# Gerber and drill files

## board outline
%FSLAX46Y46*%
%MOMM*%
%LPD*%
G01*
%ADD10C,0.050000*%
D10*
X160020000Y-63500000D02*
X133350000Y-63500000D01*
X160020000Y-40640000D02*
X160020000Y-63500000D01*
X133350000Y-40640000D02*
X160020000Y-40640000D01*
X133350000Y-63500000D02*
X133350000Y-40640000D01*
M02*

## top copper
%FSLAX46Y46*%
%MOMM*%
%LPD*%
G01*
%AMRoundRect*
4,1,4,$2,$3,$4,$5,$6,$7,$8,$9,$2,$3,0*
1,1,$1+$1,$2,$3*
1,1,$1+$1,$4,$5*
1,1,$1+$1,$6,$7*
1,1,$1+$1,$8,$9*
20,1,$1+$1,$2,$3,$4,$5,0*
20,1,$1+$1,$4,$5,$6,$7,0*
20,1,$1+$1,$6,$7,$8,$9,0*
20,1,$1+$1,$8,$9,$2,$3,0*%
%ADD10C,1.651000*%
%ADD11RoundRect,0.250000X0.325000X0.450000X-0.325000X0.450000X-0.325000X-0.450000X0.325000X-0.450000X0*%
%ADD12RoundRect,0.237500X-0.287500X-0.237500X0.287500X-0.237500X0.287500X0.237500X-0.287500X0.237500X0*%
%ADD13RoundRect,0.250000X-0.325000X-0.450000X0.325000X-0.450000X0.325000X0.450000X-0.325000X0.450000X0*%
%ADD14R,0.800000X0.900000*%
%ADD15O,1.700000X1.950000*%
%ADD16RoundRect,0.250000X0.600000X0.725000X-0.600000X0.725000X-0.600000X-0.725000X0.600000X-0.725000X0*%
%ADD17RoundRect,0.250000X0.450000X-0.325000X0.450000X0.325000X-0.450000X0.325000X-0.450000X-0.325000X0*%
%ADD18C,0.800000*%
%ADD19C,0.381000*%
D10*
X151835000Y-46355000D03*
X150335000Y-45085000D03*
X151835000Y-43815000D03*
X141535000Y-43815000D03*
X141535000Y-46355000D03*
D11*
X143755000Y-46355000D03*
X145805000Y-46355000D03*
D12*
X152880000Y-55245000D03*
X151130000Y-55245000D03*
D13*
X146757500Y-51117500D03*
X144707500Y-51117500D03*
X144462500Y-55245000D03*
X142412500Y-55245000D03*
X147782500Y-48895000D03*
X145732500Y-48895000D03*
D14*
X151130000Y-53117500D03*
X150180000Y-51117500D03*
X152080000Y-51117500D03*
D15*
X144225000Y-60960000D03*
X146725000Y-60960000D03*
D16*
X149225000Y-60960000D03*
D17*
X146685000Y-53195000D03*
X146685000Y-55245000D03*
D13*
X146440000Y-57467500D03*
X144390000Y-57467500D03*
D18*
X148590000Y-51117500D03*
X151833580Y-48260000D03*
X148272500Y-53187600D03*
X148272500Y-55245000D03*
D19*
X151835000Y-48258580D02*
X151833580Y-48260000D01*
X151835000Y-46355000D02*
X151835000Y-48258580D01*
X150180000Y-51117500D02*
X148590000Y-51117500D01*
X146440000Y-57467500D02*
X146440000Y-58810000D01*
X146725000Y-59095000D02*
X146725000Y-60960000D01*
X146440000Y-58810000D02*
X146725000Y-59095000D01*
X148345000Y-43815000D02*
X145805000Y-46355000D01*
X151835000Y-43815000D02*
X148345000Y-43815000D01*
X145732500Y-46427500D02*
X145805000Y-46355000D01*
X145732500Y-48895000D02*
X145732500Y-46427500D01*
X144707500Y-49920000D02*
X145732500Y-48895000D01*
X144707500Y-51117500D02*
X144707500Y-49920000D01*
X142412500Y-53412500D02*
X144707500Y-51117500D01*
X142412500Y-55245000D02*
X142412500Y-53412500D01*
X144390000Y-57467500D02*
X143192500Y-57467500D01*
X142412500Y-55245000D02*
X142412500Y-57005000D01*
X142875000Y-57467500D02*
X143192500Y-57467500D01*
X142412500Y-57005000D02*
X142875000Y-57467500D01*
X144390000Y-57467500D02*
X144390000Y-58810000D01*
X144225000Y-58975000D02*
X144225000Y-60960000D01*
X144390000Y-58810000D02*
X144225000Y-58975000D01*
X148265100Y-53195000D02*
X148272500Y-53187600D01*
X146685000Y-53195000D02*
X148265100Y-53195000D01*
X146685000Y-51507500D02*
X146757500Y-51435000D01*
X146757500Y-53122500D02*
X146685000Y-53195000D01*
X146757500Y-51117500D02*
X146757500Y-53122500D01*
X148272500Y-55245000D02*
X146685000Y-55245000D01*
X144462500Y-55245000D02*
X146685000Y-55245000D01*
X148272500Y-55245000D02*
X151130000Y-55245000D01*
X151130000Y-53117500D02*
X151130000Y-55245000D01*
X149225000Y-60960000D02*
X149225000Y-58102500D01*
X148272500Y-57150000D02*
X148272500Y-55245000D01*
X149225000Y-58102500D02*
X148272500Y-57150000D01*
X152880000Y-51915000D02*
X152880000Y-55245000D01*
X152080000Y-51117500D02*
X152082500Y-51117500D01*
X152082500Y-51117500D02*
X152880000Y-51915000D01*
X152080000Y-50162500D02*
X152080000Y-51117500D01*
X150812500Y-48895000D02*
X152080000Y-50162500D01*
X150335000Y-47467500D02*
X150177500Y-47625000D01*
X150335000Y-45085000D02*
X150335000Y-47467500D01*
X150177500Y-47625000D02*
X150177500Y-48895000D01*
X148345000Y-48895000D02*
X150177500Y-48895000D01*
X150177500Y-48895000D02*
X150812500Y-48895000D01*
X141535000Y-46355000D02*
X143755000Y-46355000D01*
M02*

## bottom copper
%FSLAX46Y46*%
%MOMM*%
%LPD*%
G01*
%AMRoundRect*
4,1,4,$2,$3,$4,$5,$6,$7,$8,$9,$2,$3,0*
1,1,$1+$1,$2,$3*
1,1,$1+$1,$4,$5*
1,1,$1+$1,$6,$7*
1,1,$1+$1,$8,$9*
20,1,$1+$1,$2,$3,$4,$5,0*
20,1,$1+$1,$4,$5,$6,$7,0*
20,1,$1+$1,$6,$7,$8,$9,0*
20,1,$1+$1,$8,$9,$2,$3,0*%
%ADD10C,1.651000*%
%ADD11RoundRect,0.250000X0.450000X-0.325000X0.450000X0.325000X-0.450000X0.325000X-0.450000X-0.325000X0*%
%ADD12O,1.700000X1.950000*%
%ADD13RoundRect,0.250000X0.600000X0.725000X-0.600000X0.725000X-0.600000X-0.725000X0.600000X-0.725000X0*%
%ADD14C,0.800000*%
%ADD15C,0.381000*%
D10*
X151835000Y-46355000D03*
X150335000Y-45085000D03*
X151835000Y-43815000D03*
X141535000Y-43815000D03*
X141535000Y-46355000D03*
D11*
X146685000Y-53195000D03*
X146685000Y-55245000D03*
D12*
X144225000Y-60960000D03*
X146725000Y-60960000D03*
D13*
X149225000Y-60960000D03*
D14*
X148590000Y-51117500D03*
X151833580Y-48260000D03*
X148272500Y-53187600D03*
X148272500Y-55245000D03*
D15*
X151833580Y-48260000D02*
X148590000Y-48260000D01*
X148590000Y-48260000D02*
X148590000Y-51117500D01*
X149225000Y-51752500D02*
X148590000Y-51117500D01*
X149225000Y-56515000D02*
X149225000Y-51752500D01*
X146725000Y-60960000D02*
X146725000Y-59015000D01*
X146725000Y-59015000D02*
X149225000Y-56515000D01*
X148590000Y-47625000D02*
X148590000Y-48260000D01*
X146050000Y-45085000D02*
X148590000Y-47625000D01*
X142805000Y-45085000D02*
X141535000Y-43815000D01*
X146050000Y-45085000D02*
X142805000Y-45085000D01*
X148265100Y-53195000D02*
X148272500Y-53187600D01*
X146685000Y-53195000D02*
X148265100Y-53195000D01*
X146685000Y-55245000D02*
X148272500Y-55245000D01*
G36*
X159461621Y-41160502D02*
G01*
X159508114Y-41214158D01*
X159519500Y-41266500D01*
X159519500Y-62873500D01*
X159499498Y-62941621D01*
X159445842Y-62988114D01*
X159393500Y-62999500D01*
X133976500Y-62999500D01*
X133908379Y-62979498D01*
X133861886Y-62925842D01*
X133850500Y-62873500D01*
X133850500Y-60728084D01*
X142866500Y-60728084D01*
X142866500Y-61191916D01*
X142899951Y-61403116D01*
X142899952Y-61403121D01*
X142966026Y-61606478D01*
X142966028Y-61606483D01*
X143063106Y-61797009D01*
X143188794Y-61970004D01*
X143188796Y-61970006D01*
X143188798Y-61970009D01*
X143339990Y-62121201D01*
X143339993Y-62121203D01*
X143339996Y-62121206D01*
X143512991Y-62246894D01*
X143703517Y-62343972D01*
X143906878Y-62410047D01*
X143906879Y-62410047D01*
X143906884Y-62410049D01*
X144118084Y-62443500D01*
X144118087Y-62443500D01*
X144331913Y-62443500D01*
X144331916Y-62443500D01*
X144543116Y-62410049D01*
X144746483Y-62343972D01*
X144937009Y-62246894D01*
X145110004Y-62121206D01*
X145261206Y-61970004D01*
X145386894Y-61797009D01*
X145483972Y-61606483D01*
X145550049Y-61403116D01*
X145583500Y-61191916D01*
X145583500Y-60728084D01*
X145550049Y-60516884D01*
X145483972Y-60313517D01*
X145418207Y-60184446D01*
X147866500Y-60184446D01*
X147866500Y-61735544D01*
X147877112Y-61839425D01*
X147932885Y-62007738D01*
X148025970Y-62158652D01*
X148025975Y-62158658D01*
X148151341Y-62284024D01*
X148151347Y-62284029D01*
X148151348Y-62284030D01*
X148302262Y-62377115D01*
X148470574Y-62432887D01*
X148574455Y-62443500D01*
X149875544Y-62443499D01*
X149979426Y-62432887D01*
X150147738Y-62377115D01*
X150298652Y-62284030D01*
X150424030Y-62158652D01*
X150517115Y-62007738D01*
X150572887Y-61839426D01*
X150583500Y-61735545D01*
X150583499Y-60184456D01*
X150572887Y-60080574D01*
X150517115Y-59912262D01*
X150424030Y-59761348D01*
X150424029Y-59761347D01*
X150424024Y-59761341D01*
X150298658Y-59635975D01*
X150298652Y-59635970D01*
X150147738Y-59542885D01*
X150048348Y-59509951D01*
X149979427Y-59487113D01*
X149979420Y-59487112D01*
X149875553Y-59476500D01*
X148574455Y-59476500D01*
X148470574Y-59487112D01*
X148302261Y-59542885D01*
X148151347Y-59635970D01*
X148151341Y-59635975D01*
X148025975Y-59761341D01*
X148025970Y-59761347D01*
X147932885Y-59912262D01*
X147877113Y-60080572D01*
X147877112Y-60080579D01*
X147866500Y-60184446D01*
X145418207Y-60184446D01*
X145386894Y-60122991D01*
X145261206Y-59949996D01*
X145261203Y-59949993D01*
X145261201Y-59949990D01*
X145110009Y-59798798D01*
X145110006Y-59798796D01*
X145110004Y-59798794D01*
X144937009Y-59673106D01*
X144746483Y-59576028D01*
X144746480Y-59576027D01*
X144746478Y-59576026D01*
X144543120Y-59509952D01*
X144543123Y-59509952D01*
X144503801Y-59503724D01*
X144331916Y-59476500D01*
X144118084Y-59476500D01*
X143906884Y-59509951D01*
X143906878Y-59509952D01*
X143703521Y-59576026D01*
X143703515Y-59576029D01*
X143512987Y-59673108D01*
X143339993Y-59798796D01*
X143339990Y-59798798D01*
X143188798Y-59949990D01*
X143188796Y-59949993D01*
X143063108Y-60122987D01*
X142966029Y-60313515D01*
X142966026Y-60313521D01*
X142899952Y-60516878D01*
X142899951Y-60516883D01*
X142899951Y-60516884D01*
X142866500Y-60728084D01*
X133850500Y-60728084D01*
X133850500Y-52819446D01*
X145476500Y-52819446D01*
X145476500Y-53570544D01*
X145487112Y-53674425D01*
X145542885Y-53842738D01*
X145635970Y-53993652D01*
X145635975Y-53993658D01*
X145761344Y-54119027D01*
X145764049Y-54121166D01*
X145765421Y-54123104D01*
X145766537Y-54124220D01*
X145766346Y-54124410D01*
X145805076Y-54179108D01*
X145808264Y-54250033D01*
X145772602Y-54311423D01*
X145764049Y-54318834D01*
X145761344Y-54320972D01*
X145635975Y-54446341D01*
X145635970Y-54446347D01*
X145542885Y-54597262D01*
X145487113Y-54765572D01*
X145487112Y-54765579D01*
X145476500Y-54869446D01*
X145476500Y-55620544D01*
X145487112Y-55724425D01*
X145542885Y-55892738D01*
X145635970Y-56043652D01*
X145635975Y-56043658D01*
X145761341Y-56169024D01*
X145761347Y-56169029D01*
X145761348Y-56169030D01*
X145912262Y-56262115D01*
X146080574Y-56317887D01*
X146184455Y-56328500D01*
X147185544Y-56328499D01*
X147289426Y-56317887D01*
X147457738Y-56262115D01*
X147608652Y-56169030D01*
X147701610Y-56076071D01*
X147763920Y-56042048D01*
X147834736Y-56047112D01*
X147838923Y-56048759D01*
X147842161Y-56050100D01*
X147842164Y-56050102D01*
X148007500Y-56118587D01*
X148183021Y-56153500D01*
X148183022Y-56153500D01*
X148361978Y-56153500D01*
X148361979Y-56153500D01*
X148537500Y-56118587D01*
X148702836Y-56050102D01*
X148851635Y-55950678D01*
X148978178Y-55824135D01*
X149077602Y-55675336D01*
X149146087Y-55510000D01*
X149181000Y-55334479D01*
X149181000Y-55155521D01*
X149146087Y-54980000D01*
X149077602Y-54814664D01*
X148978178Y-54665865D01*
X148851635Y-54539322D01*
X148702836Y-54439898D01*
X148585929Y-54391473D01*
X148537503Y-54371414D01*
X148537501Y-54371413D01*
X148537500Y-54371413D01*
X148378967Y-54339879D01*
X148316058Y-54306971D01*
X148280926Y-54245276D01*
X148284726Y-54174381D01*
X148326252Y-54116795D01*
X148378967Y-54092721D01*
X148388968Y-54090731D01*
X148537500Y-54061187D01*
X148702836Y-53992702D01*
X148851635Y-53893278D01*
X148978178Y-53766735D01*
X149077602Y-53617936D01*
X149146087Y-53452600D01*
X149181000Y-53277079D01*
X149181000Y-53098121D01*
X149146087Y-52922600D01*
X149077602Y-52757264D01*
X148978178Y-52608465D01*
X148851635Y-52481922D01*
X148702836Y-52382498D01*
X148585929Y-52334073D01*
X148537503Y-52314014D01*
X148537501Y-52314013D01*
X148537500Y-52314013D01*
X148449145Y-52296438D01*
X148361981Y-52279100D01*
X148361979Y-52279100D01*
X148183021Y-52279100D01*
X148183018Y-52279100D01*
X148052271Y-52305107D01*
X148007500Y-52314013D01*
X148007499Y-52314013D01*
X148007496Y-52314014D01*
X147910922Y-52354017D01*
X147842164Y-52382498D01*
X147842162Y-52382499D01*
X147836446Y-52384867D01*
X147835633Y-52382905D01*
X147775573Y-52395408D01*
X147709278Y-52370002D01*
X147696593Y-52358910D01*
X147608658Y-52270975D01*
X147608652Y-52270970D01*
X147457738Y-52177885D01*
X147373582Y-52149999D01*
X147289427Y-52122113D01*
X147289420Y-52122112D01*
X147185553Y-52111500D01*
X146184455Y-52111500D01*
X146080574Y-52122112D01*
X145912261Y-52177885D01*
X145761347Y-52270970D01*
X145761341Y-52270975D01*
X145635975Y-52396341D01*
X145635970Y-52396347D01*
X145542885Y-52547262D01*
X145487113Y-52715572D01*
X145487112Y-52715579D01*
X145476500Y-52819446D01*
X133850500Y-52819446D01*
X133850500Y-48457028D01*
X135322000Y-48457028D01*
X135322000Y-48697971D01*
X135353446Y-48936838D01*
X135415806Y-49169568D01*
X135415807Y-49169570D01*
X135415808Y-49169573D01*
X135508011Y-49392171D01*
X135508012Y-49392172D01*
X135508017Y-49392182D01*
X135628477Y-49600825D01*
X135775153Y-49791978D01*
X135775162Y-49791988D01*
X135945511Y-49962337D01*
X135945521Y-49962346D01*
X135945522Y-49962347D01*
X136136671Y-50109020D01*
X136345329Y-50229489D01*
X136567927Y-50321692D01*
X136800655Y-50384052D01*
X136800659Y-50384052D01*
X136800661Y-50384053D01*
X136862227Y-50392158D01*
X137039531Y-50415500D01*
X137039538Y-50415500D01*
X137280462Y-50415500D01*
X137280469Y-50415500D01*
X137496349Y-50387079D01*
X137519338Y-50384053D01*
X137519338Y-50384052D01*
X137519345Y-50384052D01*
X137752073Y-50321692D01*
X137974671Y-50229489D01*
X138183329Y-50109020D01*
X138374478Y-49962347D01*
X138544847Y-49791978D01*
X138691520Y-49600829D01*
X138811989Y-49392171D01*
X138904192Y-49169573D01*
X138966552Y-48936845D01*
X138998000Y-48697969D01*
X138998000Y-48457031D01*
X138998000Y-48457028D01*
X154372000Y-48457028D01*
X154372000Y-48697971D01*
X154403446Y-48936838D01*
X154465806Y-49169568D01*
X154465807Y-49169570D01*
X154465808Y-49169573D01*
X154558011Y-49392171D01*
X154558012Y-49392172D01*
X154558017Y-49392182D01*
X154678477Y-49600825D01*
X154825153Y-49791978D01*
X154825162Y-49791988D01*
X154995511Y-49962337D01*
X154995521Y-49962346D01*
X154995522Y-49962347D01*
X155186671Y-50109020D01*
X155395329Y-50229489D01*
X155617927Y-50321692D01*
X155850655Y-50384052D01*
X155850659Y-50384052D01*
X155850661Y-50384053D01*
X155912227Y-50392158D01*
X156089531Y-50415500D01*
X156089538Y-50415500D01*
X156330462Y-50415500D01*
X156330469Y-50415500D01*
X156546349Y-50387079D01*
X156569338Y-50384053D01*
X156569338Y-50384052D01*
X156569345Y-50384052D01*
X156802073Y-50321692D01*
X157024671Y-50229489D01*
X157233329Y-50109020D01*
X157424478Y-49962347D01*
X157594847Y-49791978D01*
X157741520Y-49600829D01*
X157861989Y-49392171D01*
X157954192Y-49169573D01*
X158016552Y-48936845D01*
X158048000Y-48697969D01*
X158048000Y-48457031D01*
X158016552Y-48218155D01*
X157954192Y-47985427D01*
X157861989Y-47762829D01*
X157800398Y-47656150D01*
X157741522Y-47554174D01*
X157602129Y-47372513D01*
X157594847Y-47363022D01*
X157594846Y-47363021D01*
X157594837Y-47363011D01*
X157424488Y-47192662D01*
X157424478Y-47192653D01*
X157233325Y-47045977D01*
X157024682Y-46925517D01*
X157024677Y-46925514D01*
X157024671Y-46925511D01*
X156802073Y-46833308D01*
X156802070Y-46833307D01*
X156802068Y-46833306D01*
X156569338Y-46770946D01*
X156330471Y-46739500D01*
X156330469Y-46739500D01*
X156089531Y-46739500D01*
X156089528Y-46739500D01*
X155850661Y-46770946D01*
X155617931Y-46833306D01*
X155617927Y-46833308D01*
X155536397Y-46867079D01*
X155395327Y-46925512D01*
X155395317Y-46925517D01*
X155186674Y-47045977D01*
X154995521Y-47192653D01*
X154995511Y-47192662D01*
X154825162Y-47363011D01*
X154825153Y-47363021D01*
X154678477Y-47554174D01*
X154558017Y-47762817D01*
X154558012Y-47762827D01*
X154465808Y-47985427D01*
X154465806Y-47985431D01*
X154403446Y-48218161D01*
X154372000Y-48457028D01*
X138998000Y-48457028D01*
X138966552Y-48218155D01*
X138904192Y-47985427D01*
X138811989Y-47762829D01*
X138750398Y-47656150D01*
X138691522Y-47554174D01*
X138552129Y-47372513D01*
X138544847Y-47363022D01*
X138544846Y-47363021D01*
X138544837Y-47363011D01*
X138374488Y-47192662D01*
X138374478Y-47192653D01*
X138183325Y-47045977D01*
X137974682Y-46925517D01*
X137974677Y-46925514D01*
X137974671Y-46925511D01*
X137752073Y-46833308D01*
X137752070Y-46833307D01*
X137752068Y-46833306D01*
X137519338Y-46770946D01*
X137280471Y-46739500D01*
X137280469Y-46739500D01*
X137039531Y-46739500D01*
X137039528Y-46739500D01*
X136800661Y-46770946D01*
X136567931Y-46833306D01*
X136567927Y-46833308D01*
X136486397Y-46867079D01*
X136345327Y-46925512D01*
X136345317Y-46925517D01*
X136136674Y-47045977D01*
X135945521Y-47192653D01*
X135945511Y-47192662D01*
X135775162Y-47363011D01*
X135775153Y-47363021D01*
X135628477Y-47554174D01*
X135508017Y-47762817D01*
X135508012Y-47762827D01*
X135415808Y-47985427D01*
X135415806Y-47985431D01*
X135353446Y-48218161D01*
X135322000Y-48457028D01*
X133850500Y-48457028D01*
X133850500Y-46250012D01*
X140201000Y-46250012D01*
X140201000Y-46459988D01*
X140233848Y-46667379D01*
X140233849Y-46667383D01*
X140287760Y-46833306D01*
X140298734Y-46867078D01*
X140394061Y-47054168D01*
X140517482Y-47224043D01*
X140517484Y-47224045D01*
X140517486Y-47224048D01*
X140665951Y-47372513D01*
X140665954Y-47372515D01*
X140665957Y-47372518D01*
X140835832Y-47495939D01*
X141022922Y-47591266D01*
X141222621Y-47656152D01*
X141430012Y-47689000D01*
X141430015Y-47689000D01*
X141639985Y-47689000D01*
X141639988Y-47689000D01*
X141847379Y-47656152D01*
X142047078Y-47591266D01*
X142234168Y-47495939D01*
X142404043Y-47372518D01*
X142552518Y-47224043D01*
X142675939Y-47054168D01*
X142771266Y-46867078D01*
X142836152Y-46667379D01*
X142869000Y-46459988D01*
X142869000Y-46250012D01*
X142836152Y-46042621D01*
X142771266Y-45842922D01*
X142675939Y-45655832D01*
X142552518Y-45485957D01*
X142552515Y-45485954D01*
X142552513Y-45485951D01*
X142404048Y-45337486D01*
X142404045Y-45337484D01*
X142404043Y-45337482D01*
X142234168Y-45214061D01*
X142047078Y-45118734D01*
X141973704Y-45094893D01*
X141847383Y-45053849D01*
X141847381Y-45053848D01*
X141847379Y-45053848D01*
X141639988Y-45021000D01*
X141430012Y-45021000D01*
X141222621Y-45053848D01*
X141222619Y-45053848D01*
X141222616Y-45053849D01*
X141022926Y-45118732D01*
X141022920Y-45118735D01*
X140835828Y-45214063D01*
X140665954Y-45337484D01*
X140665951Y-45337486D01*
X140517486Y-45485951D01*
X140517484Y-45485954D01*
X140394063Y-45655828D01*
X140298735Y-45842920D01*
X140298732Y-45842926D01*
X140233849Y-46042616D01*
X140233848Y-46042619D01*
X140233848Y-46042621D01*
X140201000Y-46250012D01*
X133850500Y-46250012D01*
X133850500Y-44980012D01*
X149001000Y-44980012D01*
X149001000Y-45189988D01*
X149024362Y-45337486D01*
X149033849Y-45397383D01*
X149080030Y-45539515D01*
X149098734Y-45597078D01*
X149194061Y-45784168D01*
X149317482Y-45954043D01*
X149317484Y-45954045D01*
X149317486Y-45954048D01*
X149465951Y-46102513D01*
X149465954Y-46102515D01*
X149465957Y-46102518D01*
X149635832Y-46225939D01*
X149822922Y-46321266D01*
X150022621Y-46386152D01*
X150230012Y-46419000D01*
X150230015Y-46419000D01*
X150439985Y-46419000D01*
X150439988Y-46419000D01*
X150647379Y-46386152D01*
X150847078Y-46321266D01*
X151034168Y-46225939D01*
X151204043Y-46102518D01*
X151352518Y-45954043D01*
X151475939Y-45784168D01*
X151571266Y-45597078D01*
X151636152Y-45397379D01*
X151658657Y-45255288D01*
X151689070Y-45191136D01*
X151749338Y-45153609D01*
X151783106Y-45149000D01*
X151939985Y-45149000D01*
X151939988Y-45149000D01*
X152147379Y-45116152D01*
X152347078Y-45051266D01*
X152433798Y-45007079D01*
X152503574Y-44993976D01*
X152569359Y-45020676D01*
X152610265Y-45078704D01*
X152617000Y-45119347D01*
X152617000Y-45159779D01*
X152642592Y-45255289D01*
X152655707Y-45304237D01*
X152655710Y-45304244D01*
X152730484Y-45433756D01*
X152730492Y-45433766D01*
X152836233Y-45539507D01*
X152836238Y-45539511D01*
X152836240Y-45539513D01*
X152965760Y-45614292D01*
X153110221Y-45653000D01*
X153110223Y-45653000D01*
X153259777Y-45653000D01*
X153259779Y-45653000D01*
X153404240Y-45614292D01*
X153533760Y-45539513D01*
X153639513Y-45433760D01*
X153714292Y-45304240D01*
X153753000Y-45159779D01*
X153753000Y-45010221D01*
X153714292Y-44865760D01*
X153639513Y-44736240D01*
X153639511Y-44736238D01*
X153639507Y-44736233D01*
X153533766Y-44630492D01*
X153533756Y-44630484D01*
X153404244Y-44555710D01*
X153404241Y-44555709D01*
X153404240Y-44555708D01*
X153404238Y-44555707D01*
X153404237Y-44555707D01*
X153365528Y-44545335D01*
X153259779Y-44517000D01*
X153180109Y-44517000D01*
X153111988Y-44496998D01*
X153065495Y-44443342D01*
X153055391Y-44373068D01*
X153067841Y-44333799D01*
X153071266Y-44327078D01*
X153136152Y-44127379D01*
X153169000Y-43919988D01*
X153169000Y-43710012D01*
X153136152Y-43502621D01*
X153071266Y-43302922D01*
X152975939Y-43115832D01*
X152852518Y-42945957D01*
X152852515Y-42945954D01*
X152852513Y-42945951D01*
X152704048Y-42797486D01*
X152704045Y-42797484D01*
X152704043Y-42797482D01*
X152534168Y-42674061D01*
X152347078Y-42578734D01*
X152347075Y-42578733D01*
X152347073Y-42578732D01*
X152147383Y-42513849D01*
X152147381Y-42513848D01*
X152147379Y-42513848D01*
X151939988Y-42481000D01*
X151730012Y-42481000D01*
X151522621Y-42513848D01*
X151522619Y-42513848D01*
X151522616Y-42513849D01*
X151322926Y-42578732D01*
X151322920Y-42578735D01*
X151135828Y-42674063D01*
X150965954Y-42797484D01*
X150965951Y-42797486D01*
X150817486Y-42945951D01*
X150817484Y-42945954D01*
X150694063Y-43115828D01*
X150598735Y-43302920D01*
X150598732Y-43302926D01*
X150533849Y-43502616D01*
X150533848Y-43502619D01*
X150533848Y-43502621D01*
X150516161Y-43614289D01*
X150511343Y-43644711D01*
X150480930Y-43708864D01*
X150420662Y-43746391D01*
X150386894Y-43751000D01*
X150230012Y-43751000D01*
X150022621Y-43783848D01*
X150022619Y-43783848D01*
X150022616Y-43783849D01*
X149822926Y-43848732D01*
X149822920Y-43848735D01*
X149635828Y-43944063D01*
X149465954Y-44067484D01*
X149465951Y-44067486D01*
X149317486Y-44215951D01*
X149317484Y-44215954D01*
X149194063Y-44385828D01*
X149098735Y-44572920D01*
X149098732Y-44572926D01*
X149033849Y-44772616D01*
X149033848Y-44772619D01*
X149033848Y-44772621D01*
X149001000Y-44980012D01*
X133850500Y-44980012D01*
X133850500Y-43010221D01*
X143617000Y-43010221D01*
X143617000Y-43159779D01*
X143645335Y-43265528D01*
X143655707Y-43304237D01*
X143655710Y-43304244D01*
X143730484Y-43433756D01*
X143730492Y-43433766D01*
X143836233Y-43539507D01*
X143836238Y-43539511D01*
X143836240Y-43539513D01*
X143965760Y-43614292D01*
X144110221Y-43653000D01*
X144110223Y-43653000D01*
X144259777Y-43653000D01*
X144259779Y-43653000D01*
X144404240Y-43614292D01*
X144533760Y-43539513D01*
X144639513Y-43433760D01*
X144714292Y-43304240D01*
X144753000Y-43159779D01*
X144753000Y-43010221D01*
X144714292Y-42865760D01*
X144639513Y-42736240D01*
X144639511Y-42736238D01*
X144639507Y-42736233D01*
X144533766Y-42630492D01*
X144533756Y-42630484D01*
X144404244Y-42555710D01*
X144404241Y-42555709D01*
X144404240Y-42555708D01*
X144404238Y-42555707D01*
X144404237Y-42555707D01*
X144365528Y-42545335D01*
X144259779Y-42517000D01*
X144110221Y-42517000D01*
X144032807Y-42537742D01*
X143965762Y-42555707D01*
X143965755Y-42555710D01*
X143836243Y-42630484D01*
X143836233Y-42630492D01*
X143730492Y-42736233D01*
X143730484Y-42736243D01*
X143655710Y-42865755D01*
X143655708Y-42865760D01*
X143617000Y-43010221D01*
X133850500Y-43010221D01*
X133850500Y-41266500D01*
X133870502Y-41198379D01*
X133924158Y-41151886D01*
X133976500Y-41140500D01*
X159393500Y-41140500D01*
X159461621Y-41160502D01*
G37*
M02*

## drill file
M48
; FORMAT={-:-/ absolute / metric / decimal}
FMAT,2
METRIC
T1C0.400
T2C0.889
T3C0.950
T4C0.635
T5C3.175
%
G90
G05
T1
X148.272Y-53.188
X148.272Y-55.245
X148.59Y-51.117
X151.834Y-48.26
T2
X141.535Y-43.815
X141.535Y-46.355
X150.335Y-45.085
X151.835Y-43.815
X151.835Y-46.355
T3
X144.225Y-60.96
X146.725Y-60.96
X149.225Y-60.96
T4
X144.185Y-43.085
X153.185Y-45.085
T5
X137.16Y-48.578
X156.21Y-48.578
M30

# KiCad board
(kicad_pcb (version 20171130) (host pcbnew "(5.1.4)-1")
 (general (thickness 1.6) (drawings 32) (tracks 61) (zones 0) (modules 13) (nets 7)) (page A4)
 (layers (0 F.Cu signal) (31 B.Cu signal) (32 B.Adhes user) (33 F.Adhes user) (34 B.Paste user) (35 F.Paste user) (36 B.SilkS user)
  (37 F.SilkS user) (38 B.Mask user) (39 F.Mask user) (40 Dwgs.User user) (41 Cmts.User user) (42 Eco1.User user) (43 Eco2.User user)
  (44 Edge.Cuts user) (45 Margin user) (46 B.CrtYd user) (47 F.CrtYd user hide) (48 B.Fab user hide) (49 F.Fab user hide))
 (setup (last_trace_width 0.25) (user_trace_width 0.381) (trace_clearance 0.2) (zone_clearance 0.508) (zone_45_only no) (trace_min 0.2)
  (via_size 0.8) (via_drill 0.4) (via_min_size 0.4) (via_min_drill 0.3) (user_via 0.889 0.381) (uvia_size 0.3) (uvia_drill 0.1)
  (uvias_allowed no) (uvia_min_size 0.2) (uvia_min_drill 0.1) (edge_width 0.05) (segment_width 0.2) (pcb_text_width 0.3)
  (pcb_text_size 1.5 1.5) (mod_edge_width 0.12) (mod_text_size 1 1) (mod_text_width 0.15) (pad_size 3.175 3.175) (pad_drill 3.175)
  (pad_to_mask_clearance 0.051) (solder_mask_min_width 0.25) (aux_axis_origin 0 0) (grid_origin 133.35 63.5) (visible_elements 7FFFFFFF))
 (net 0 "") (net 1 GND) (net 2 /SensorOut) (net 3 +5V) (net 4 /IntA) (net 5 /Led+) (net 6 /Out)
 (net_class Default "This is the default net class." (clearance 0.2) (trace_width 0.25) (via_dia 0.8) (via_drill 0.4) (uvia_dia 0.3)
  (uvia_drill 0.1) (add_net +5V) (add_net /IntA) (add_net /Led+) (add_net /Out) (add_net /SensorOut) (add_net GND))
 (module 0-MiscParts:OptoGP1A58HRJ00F (layer B.Cu) (at 146.685 45.085 180)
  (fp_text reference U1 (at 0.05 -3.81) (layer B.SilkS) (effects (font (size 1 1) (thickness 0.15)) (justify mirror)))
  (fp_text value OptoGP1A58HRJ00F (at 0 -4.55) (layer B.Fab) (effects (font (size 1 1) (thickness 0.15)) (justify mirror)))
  (pad "" np_thru_hole circle (at 2.5 2 180) (size 0.635 0.635) (drill 0.635) (layers *.Cu *.Mask))
  (pad "" np_thru_hole circle (at -6.5 0 180) (size 0.635 0.635) (drill 0.635) (layers *.Cu *.Mask))
  (pad 5 thru_hole circle (at -5.15 -1.27 180) (size 1.651 1.651) (drill 0.889) (layers *.Cu *.Mask) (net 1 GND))
  (pad 4 thru_hole circle (at -3.65 0 180) (size 1.651 1.651) (drill 0.889) (layers *.Cu *.Mask) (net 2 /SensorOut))
  (pad 3 thru_hole circle (at -5.15 1.27 180) (size 1.651 1.651) (drill 0.889) (layers *.Cu *.Mask) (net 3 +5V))
  (pad 2 thru_hole circle (at 5.15 1.27 180) (size 1.651 1.651) (drill 0.889) (layers *.Cu *.Mask) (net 1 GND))
  (pad 1 thru_hole circle (at 5.15 -1.27 180) (size 1.651 1.651) (drill 0.889) (layers *.Cu *.Mask) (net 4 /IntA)))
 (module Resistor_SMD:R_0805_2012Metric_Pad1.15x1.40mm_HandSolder (layer F.Cu) (at 144.78 46.355 180)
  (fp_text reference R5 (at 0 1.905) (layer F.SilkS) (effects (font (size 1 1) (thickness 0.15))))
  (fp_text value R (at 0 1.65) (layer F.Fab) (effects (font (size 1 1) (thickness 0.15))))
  (pad 2 smd roundrect (at 1.025 0 180) (size 1.15 1.4) (layers F.Cu F.Paste F.Mask) (roundrect_rratio 0.217391) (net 4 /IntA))
  (pad 1 smd roundrect (at -1.025 0 180) (size 1.15 1.4) (layers F.Cu F.Paste F.Mask) (roundrect_rratio 0.217391) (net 3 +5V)))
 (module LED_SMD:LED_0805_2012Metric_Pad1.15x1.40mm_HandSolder (layer B.Cu) (at 146.685 54.22 90)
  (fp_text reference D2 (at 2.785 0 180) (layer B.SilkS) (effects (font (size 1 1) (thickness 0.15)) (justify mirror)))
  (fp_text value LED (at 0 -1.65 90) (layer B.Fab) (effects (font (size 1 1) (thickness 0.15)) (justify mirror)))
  (pad 2 smd roundrect (at 1.025 0 90) (size 1.15 1.4) (layers B.Cu B.Paste B.Mask) (roundrect_rratio 0.217391) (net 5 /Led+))
  (pad 1 smd roundrect (at -1.025 0 90) (size 1.15 1.4) (layers B.Cu B.Paste B.Mask) (roundrect_rratio 0.217391) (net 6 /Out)))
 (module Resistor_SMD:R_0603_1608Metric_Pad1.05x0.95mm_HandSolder (layer F.Cu) (at 152.005 55.245)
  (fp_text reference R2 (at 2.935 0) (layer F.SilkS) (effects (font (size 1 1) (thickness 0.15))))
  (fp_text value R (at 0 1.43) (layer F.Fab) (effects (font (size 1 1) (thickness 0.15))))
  (pad 2 smd roundrect (at 0.875 0) (size 1.05 0.95) (layers F.Cu F.Paste F.Mask) (roundrect_rratio 0.25) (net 2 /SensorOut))
  (pad 1 smd roundrect (at -0.875 0) (size 1.05 0.95) (layers F.Cu F.Paste F.Mask) (roundrect_rratio 0.25) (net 6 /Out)))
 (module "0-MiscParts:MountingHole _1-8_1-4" (layer F.Cu) (at 156.21 48.5775)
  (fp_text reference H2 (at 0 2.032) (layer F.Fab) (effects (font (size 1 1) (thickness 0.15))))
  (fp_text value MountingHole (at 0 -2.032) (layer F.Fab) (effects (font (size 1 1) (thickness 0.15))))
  (pad "" np_thru_hole circle (at 0 0) (size 3.175 3.175) (drill 3.175) (layers *.Cu *.Mask)))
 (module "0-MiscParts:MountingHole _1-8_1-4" (layer F.Cu) (at 137.16 48.5775)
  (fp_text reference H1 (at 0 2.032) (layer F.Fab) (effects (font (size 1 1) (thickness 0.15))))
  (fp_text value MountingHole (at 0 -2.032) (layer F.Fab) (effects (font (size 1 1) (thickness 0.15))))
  (pad "" np_thru_hole circle (at 0 0) (size 3.175 3.175) (drill 3.175) (layers *.Cu *.Mask)))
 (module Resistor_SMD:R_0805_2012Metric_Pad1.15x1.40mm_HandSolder (layer F.Cu) (at 145.7325 51.1175)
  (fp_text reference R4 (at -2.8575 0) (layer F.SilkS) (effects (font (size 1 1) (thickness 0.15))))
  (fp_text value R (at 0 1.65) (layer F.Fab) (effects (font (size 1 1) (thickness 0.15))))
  (pad 2 smd roundrect (at 1.025 0) (size 1.15 1.4) (layers F.Cu F.Paste F.Mask) (roundrect_rratio 0.217391) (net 5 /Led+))
  (pad 1 smd roundrect (at -1.025 0) (size 1.15 1.4) (layers F.Cu F.Paste F.Mask) (roundrect_rratio 0.217391) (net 3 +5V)))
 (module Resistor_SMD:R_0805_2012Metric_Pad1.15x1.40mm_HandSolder (layer F.Cu) (at 143.4375 55.245)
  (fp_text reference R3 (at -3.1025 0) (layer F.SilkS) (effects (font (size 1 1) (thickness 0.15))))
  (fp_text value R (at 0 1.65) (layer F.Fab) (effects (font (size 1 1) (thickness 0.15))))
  (pad 2 smd roundrect (at 1.025 0) (size 1.15 1.4) (layers F.Cu F.Paste F.Mask) (roundrect_rratio 0.217391) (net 6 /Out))
  (pad 1 smd roundrect (at -1.025 0) (size 1.15 1.4) (layers F.Cu F.Paste F.Mask) (roundrect_rratio 0.217391) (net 3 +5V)))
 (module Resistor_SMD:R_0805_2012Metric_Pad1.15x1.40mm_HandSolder (layer F.Cu) (at 146.7575 48.895)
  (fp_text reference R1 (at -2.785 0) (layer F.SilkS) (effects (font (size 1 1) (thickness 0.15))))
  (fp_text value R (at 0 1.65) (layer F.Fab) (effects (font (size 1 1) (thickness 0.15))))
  (pad 2 smd roundrect (at 1.025 0) (size 1.15 1.4) (layers F.Cu F.Paste F.Mask) (roundrect_rratio 0.217391) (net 2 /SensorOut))
  (pad 1 smd roundrect (at -1.025 0) (size 1.15 1.4) (layers F.Cu F.Paste F.Mask) (roundrect_rratio 0.217391) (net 3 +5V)))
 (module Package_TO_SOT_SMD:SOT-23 (layer F.Cu) (at 151.13 52.1175 270)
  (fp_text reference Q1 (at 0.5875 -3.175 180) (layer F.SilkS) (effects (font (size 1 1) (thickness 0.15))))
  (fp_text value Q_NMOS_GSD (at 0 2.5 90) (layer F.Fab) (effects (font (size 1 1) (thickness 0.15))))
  (pad 3 smd rect (at 1 0 270) (size 0.9 0.8) (layers F.Cu F.Paste F.Mask) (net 6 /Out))
  (pad 2 smd rect (at -1 0.95 270) (size 0.9 0.8) (layers F.Cu F.Paste F.Mask) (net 1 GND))
  (pad 1 smd rect (at -1 -0.95 270) (size 0.9 0.8) (layers F.Cu F.Paste F.Mask) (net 2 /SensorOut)))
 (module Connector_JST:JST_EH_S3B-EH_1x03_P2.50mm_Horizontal (layer F.Cu) (at 149.225 60.96 180)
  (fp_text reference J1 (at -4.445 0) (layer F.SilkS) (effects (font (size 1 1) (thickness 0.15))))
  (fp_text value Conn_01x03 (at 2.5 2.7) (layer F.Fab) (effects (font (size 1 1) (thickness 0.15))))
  (pad 3 thru_hole oval (at 5 0 180) (size 1.7 1.95) (drill 0.95) (layers *.Cu *.Mask) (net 3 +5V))
  (pad 2 thru_hole oval (at 2.5 0 180) (size 1.7 1.95) (drill 0.95) (layers *.Cu *.Mask) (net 1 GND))
  (pad 1 thru_hole roundrect (at 0 0 180) (size 1.7 1.95) (drill 0.95) (layers *.Cu *.Mask) (roundrect_rratio 0.147059) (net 6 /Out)))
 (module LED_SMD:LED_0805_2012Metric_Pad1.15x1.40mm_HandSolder (layer F.Cu) (at 146.685 54.22 90)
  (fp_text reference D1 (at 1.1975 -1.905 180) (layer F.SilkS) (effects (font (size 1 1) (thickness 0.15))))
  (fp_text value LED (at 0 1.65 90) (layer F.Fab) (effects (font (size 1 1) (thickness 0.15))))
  (pad 2 smd roundrect (at 1.025 0 90) (size 1.15 1.4) (layers F.Cu F.Paste F.Mask) (roundrect_rratio 0.217391) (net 5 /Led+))
  (pad 1 smd roundrect (at -1.025 0 90) (size 1.15 1.4) (layers F.Cu F.Paste F.Mask) (roundrect_rratio 0.217391) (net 6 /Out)))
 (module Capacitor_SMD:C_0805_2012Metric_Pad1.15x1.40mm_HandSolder (layer F.Cu) (at 145.415 57.4675)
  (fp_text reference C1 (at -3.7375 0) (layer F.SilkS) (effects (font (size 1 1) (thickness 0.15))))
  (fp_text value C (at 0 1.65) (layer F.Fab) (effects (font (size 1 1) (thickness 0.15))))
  (pad 2 smd roundrect (at 1.025 0) (size 1.15 1.4) (layers F.Cu F.Paste F.Mask) (roundrect_rratio 0.217391) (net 1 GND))
  (pad 1 smd roundrect (at -1.025 0) (size 1.15 1.4) (layers F.Cu F.Paste F.Mask) (roundrect_rratio 0.217391) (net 3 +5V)))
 (gr_line (start 160.02 63.5) (end 133.35 63.5) (layer Edge.Cuts) (width 0.05))
 (gr_line (start 160.02 40.64) (end 160.02 63.5) (layer Edge.Cuts) (width 0.05))
 (gr_line (start 133.35 40.64) (end 160.02 40.64) (layer Edge.Cuts) (width 0.05))
 (gr_line (start 133.35 63.5) (end 133.35 40.64) (layer Edge.Cuts) (width 0.05))
 (via (at 148.59 51.1175) (size 0.8) (drill 0.4) (layers F.Cu B.Cu) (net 1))
 (via (at 151.83358 48.26) (size 0.8) (drill 0.4) (layers F.Cu B.Cu) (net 1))
 (segment (start 151.835 48.25858) (end 151.83358 48.26) (width 0.381) (layer F.Cu) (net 1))
 (segment (start 151.835 46.355) (end 151.835 48.25858) (width 0.381) (layer F.Cu) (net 1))
 (segment (start 150.18 51.1175) (end 148.59 51.1175) (width 0.381) (layer F.Cu) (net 1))
 (segment (start 151.83358 48.26) (end 148.59 48.26) (width 0.381) (layer B.Cu) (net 1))
 (segment (start 148.59 48.26) (end 148.59 51.1175) (width 0.381) (layer B.Cu) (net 1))
 (segment (start 149.225 51.7525) (end 148.59 51.1175) (width 0.381) (layer B.Cu) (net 1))
 (segment (start 149.225 56.515) (end 149.225 51.7525) (width 0.381) (layer B.Cu) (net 1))
 (segment (start 146.725 60.96) (end 146.725 59.015) (width 0.381) (layer B.Cu) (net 1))
 (segment (start 146.725 59.015) (end 149.225 56.515) (width 0.381) (layer B.Cu) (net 1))
 (segment (start 146.44 57.4675) (end 146.44 58.81) (width 0.381) (layer F.Cu) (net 1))
 (segment (start 146.725 59.095) (end 146.725 60.96) (width 0.381) (layer F.Cu) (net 1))
 (segment (start 146.44 58.81) (end 146.725 59.095) (width 0.381) (layer F.Cu) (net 1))
 (segment (start 148.59 47.625) (end 148.59 48.26) (width 0.381) (layer B.Cu) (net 1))
 (segment (start 146.05 45.085) (end 148.59 47.625) (width 0.381) (layer B.Cu) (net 1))
 (segment (start 142.805 45.085) (end 141.535 43.815) (width 0.381) (layer B.Cu) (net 1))
 (segment (start 146.05 45.085) (end 142.805 45.085) (width 0.381) (layer B.Cu) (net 1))
 (segment (start 148.345 43.815) (end 145.805 46.355) (width 0.381) (layer F.Cu) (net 3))
 (segment (start 151.835 43.815) (end 148.345 43.815) (width 0.381) (layer F.Cu) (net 3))
 (segment (start 145.7325 46.4275) (end 145.805 46.355) (width 0.381) (layer F.Cu) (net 3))
 (segment (start 145.7325 48.895) (end 145.7325 46.4275) (width 0.381) (layer F.Cu) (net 3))
 (segment (start 144.7075 49.92) (end 145.7325 48.895) (width 0.381) (layer F.Cu) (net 3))
 (segment (start 144.7075 51.1175) (end 144.7075 49.92) (width 0.381) (layer F.Cu) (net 3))
 (segment (start 142.4125 53.4125) (end 144.7075 51.1175) (width 0.381) (layer F.Cu) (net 3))
 (segment (start 142.4125 55.245) (end 142.4125 53.4125) (width 0.381) (layer F.Cu) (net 3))
 (segment (start 144.39 57.4675) (end 143.1925 57.4675) (width 0.381) (layer F.Cu) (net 3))
 (segment (start 142.4125 55.245) (end 142.4125 57.005) (width 0.381) (layer F.Cu) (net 3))
 (segment (start 142.875 57.4675) (end 143.1925 57.4675) (width 0.381) (layer F.Cu) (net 3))
 (segment (start 142.4125 57.005) (end 142.875 57.4675) (width 0.381) (layer F.Cu) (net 3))
 (segment (start 144.39 57.4675) (end 144.39 58.81) (width 0.381) (layer F.Cu) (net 3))
 (segment (start 144.225 58.975) (end 144.225 60.96) (width 0.381) (layer F.Cu) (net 3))
 (segment (start 144.39 58.81) (end 144.225 58.975) (width 0.381) (layer F.Cu) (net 3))
 (via (at 148.2725 53.1876) (size 0.8) (drill 0.4) (layers F.Cu B.Cu) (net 5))
 (segment (start 148.2651 53.195) (end 148.2725 53.1876) (width 0.381) (layer F.Cu) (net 5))
 (segment (start 146.685 53.195) (end 148.2651 53.195) (width 0.381) (layer F.Cu) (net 5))
 (segment (start 148.2651 53.195) (end 148.2725 53.1876) (width 0.381) (layer B.Cu) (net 5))
 (segment (start 146.685 53.195) (end 148.2651 53.195) (width 0.381) (layer B.Cu) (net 5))
 (segment (start 146.685 51.5075) (end 146.7575 51.435) (width 0.381) (layer F.Cu) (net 5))
 (segment (start 146.7575 53.1225) (end 146.685 53.195) (width 0.381) (layer F.Cu) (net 5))
 (segment (start 146.7575 51.1175) (end 146.7575 53.1225) (width 0.381) (layer F.Cu) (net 5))
 (via (at 148.2725 55.245) (size 0.8) (drill 0.4) (layers F.Cu B.Cu) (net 6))
 (segment (start 148.2725 55.245) (end 146.685 55.245) (width 0.381) (layer F.Cu) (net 6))
 (segment (start 146.685 55.245) (end 148.2725 55.245) (width 0.381) (layer B.Cu) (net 6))
 (segment (start 144.4625 55.245) (end 146.685 55.245) (width 0.381) (layer F.Cu) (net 6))
 (segment (start 148.2725 55.245) (end 151.13 55.245) (width 0.381) (layer F.Cu) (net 6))
 (segment (start 151.13 53.1175) (end 151.13 55.245) (width 0.381) (layer F.Cu) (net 6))
 (segment (start 149.225 60.96) (end 149.225 58.1025) (width 0.381) (layer F.Cu) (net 6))
 (segment (start 148.2725 57.15) (end 148.2725 55.245) (width 0.381) (layer F.Cu) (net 6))
 (segment (start 149.225 58.1025) (end 148.2725 57.15) (width 0.381) (layer F.Cu) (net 6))
 (segment (start 152.88 51.915) (end 152.88 55.245) (width 0.381) (layer F.Cu) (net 2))
 (segment (start 152.08 51.1175) (end 152.0825 51.1175) (width 0.381) (layer F.Cu) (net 2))
 (segment (start 152.0825 51.1175) (end 152.88 51.915) (width 0.381) (layer F.Cu) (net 2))
 (segment (start 152.08 50.1625) (end 152.08 51.1175) (width 0.381) (layer F.Cu) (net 2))
 (segment (start 150.8125 48.895) (end 152.08 50.1625) (width 0.381) (layer F.Cu) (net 2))
 (segment (start 150.335 47.4675) (end 150.1775 47.625) (width 0.381) (layer F.Cu) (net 2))
 (segment (start 150.335 45.085) (end 150.335 47.4675) (width 0.381) (layer F.Cu) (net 2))
 (segment (start 150.1775 47.625) (end 150.1775 48.895) (width 0.381) (layer F.Cu) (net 2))
 (segment (start 148.345 48.895) (end 150.1775 48.895) (width 0.381) (layer F.Cu) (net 2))
 (segment (start 150.1775 48.895) (end 150.8125 48.895) (width 0.381) (layer F.Cu) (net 2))
 (segment (start 141.535 46.355) (end 143.755 46.355) (width 0.381) (layer F.Cu) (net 4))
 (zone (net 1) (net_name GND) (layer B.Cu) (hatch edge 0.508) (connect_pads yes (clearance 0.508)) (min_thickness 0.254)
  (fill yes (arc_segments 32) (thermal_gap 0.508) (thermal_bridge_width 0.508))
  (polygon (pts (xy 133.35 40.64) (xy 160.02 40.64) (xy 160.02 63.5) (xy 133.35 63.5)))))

